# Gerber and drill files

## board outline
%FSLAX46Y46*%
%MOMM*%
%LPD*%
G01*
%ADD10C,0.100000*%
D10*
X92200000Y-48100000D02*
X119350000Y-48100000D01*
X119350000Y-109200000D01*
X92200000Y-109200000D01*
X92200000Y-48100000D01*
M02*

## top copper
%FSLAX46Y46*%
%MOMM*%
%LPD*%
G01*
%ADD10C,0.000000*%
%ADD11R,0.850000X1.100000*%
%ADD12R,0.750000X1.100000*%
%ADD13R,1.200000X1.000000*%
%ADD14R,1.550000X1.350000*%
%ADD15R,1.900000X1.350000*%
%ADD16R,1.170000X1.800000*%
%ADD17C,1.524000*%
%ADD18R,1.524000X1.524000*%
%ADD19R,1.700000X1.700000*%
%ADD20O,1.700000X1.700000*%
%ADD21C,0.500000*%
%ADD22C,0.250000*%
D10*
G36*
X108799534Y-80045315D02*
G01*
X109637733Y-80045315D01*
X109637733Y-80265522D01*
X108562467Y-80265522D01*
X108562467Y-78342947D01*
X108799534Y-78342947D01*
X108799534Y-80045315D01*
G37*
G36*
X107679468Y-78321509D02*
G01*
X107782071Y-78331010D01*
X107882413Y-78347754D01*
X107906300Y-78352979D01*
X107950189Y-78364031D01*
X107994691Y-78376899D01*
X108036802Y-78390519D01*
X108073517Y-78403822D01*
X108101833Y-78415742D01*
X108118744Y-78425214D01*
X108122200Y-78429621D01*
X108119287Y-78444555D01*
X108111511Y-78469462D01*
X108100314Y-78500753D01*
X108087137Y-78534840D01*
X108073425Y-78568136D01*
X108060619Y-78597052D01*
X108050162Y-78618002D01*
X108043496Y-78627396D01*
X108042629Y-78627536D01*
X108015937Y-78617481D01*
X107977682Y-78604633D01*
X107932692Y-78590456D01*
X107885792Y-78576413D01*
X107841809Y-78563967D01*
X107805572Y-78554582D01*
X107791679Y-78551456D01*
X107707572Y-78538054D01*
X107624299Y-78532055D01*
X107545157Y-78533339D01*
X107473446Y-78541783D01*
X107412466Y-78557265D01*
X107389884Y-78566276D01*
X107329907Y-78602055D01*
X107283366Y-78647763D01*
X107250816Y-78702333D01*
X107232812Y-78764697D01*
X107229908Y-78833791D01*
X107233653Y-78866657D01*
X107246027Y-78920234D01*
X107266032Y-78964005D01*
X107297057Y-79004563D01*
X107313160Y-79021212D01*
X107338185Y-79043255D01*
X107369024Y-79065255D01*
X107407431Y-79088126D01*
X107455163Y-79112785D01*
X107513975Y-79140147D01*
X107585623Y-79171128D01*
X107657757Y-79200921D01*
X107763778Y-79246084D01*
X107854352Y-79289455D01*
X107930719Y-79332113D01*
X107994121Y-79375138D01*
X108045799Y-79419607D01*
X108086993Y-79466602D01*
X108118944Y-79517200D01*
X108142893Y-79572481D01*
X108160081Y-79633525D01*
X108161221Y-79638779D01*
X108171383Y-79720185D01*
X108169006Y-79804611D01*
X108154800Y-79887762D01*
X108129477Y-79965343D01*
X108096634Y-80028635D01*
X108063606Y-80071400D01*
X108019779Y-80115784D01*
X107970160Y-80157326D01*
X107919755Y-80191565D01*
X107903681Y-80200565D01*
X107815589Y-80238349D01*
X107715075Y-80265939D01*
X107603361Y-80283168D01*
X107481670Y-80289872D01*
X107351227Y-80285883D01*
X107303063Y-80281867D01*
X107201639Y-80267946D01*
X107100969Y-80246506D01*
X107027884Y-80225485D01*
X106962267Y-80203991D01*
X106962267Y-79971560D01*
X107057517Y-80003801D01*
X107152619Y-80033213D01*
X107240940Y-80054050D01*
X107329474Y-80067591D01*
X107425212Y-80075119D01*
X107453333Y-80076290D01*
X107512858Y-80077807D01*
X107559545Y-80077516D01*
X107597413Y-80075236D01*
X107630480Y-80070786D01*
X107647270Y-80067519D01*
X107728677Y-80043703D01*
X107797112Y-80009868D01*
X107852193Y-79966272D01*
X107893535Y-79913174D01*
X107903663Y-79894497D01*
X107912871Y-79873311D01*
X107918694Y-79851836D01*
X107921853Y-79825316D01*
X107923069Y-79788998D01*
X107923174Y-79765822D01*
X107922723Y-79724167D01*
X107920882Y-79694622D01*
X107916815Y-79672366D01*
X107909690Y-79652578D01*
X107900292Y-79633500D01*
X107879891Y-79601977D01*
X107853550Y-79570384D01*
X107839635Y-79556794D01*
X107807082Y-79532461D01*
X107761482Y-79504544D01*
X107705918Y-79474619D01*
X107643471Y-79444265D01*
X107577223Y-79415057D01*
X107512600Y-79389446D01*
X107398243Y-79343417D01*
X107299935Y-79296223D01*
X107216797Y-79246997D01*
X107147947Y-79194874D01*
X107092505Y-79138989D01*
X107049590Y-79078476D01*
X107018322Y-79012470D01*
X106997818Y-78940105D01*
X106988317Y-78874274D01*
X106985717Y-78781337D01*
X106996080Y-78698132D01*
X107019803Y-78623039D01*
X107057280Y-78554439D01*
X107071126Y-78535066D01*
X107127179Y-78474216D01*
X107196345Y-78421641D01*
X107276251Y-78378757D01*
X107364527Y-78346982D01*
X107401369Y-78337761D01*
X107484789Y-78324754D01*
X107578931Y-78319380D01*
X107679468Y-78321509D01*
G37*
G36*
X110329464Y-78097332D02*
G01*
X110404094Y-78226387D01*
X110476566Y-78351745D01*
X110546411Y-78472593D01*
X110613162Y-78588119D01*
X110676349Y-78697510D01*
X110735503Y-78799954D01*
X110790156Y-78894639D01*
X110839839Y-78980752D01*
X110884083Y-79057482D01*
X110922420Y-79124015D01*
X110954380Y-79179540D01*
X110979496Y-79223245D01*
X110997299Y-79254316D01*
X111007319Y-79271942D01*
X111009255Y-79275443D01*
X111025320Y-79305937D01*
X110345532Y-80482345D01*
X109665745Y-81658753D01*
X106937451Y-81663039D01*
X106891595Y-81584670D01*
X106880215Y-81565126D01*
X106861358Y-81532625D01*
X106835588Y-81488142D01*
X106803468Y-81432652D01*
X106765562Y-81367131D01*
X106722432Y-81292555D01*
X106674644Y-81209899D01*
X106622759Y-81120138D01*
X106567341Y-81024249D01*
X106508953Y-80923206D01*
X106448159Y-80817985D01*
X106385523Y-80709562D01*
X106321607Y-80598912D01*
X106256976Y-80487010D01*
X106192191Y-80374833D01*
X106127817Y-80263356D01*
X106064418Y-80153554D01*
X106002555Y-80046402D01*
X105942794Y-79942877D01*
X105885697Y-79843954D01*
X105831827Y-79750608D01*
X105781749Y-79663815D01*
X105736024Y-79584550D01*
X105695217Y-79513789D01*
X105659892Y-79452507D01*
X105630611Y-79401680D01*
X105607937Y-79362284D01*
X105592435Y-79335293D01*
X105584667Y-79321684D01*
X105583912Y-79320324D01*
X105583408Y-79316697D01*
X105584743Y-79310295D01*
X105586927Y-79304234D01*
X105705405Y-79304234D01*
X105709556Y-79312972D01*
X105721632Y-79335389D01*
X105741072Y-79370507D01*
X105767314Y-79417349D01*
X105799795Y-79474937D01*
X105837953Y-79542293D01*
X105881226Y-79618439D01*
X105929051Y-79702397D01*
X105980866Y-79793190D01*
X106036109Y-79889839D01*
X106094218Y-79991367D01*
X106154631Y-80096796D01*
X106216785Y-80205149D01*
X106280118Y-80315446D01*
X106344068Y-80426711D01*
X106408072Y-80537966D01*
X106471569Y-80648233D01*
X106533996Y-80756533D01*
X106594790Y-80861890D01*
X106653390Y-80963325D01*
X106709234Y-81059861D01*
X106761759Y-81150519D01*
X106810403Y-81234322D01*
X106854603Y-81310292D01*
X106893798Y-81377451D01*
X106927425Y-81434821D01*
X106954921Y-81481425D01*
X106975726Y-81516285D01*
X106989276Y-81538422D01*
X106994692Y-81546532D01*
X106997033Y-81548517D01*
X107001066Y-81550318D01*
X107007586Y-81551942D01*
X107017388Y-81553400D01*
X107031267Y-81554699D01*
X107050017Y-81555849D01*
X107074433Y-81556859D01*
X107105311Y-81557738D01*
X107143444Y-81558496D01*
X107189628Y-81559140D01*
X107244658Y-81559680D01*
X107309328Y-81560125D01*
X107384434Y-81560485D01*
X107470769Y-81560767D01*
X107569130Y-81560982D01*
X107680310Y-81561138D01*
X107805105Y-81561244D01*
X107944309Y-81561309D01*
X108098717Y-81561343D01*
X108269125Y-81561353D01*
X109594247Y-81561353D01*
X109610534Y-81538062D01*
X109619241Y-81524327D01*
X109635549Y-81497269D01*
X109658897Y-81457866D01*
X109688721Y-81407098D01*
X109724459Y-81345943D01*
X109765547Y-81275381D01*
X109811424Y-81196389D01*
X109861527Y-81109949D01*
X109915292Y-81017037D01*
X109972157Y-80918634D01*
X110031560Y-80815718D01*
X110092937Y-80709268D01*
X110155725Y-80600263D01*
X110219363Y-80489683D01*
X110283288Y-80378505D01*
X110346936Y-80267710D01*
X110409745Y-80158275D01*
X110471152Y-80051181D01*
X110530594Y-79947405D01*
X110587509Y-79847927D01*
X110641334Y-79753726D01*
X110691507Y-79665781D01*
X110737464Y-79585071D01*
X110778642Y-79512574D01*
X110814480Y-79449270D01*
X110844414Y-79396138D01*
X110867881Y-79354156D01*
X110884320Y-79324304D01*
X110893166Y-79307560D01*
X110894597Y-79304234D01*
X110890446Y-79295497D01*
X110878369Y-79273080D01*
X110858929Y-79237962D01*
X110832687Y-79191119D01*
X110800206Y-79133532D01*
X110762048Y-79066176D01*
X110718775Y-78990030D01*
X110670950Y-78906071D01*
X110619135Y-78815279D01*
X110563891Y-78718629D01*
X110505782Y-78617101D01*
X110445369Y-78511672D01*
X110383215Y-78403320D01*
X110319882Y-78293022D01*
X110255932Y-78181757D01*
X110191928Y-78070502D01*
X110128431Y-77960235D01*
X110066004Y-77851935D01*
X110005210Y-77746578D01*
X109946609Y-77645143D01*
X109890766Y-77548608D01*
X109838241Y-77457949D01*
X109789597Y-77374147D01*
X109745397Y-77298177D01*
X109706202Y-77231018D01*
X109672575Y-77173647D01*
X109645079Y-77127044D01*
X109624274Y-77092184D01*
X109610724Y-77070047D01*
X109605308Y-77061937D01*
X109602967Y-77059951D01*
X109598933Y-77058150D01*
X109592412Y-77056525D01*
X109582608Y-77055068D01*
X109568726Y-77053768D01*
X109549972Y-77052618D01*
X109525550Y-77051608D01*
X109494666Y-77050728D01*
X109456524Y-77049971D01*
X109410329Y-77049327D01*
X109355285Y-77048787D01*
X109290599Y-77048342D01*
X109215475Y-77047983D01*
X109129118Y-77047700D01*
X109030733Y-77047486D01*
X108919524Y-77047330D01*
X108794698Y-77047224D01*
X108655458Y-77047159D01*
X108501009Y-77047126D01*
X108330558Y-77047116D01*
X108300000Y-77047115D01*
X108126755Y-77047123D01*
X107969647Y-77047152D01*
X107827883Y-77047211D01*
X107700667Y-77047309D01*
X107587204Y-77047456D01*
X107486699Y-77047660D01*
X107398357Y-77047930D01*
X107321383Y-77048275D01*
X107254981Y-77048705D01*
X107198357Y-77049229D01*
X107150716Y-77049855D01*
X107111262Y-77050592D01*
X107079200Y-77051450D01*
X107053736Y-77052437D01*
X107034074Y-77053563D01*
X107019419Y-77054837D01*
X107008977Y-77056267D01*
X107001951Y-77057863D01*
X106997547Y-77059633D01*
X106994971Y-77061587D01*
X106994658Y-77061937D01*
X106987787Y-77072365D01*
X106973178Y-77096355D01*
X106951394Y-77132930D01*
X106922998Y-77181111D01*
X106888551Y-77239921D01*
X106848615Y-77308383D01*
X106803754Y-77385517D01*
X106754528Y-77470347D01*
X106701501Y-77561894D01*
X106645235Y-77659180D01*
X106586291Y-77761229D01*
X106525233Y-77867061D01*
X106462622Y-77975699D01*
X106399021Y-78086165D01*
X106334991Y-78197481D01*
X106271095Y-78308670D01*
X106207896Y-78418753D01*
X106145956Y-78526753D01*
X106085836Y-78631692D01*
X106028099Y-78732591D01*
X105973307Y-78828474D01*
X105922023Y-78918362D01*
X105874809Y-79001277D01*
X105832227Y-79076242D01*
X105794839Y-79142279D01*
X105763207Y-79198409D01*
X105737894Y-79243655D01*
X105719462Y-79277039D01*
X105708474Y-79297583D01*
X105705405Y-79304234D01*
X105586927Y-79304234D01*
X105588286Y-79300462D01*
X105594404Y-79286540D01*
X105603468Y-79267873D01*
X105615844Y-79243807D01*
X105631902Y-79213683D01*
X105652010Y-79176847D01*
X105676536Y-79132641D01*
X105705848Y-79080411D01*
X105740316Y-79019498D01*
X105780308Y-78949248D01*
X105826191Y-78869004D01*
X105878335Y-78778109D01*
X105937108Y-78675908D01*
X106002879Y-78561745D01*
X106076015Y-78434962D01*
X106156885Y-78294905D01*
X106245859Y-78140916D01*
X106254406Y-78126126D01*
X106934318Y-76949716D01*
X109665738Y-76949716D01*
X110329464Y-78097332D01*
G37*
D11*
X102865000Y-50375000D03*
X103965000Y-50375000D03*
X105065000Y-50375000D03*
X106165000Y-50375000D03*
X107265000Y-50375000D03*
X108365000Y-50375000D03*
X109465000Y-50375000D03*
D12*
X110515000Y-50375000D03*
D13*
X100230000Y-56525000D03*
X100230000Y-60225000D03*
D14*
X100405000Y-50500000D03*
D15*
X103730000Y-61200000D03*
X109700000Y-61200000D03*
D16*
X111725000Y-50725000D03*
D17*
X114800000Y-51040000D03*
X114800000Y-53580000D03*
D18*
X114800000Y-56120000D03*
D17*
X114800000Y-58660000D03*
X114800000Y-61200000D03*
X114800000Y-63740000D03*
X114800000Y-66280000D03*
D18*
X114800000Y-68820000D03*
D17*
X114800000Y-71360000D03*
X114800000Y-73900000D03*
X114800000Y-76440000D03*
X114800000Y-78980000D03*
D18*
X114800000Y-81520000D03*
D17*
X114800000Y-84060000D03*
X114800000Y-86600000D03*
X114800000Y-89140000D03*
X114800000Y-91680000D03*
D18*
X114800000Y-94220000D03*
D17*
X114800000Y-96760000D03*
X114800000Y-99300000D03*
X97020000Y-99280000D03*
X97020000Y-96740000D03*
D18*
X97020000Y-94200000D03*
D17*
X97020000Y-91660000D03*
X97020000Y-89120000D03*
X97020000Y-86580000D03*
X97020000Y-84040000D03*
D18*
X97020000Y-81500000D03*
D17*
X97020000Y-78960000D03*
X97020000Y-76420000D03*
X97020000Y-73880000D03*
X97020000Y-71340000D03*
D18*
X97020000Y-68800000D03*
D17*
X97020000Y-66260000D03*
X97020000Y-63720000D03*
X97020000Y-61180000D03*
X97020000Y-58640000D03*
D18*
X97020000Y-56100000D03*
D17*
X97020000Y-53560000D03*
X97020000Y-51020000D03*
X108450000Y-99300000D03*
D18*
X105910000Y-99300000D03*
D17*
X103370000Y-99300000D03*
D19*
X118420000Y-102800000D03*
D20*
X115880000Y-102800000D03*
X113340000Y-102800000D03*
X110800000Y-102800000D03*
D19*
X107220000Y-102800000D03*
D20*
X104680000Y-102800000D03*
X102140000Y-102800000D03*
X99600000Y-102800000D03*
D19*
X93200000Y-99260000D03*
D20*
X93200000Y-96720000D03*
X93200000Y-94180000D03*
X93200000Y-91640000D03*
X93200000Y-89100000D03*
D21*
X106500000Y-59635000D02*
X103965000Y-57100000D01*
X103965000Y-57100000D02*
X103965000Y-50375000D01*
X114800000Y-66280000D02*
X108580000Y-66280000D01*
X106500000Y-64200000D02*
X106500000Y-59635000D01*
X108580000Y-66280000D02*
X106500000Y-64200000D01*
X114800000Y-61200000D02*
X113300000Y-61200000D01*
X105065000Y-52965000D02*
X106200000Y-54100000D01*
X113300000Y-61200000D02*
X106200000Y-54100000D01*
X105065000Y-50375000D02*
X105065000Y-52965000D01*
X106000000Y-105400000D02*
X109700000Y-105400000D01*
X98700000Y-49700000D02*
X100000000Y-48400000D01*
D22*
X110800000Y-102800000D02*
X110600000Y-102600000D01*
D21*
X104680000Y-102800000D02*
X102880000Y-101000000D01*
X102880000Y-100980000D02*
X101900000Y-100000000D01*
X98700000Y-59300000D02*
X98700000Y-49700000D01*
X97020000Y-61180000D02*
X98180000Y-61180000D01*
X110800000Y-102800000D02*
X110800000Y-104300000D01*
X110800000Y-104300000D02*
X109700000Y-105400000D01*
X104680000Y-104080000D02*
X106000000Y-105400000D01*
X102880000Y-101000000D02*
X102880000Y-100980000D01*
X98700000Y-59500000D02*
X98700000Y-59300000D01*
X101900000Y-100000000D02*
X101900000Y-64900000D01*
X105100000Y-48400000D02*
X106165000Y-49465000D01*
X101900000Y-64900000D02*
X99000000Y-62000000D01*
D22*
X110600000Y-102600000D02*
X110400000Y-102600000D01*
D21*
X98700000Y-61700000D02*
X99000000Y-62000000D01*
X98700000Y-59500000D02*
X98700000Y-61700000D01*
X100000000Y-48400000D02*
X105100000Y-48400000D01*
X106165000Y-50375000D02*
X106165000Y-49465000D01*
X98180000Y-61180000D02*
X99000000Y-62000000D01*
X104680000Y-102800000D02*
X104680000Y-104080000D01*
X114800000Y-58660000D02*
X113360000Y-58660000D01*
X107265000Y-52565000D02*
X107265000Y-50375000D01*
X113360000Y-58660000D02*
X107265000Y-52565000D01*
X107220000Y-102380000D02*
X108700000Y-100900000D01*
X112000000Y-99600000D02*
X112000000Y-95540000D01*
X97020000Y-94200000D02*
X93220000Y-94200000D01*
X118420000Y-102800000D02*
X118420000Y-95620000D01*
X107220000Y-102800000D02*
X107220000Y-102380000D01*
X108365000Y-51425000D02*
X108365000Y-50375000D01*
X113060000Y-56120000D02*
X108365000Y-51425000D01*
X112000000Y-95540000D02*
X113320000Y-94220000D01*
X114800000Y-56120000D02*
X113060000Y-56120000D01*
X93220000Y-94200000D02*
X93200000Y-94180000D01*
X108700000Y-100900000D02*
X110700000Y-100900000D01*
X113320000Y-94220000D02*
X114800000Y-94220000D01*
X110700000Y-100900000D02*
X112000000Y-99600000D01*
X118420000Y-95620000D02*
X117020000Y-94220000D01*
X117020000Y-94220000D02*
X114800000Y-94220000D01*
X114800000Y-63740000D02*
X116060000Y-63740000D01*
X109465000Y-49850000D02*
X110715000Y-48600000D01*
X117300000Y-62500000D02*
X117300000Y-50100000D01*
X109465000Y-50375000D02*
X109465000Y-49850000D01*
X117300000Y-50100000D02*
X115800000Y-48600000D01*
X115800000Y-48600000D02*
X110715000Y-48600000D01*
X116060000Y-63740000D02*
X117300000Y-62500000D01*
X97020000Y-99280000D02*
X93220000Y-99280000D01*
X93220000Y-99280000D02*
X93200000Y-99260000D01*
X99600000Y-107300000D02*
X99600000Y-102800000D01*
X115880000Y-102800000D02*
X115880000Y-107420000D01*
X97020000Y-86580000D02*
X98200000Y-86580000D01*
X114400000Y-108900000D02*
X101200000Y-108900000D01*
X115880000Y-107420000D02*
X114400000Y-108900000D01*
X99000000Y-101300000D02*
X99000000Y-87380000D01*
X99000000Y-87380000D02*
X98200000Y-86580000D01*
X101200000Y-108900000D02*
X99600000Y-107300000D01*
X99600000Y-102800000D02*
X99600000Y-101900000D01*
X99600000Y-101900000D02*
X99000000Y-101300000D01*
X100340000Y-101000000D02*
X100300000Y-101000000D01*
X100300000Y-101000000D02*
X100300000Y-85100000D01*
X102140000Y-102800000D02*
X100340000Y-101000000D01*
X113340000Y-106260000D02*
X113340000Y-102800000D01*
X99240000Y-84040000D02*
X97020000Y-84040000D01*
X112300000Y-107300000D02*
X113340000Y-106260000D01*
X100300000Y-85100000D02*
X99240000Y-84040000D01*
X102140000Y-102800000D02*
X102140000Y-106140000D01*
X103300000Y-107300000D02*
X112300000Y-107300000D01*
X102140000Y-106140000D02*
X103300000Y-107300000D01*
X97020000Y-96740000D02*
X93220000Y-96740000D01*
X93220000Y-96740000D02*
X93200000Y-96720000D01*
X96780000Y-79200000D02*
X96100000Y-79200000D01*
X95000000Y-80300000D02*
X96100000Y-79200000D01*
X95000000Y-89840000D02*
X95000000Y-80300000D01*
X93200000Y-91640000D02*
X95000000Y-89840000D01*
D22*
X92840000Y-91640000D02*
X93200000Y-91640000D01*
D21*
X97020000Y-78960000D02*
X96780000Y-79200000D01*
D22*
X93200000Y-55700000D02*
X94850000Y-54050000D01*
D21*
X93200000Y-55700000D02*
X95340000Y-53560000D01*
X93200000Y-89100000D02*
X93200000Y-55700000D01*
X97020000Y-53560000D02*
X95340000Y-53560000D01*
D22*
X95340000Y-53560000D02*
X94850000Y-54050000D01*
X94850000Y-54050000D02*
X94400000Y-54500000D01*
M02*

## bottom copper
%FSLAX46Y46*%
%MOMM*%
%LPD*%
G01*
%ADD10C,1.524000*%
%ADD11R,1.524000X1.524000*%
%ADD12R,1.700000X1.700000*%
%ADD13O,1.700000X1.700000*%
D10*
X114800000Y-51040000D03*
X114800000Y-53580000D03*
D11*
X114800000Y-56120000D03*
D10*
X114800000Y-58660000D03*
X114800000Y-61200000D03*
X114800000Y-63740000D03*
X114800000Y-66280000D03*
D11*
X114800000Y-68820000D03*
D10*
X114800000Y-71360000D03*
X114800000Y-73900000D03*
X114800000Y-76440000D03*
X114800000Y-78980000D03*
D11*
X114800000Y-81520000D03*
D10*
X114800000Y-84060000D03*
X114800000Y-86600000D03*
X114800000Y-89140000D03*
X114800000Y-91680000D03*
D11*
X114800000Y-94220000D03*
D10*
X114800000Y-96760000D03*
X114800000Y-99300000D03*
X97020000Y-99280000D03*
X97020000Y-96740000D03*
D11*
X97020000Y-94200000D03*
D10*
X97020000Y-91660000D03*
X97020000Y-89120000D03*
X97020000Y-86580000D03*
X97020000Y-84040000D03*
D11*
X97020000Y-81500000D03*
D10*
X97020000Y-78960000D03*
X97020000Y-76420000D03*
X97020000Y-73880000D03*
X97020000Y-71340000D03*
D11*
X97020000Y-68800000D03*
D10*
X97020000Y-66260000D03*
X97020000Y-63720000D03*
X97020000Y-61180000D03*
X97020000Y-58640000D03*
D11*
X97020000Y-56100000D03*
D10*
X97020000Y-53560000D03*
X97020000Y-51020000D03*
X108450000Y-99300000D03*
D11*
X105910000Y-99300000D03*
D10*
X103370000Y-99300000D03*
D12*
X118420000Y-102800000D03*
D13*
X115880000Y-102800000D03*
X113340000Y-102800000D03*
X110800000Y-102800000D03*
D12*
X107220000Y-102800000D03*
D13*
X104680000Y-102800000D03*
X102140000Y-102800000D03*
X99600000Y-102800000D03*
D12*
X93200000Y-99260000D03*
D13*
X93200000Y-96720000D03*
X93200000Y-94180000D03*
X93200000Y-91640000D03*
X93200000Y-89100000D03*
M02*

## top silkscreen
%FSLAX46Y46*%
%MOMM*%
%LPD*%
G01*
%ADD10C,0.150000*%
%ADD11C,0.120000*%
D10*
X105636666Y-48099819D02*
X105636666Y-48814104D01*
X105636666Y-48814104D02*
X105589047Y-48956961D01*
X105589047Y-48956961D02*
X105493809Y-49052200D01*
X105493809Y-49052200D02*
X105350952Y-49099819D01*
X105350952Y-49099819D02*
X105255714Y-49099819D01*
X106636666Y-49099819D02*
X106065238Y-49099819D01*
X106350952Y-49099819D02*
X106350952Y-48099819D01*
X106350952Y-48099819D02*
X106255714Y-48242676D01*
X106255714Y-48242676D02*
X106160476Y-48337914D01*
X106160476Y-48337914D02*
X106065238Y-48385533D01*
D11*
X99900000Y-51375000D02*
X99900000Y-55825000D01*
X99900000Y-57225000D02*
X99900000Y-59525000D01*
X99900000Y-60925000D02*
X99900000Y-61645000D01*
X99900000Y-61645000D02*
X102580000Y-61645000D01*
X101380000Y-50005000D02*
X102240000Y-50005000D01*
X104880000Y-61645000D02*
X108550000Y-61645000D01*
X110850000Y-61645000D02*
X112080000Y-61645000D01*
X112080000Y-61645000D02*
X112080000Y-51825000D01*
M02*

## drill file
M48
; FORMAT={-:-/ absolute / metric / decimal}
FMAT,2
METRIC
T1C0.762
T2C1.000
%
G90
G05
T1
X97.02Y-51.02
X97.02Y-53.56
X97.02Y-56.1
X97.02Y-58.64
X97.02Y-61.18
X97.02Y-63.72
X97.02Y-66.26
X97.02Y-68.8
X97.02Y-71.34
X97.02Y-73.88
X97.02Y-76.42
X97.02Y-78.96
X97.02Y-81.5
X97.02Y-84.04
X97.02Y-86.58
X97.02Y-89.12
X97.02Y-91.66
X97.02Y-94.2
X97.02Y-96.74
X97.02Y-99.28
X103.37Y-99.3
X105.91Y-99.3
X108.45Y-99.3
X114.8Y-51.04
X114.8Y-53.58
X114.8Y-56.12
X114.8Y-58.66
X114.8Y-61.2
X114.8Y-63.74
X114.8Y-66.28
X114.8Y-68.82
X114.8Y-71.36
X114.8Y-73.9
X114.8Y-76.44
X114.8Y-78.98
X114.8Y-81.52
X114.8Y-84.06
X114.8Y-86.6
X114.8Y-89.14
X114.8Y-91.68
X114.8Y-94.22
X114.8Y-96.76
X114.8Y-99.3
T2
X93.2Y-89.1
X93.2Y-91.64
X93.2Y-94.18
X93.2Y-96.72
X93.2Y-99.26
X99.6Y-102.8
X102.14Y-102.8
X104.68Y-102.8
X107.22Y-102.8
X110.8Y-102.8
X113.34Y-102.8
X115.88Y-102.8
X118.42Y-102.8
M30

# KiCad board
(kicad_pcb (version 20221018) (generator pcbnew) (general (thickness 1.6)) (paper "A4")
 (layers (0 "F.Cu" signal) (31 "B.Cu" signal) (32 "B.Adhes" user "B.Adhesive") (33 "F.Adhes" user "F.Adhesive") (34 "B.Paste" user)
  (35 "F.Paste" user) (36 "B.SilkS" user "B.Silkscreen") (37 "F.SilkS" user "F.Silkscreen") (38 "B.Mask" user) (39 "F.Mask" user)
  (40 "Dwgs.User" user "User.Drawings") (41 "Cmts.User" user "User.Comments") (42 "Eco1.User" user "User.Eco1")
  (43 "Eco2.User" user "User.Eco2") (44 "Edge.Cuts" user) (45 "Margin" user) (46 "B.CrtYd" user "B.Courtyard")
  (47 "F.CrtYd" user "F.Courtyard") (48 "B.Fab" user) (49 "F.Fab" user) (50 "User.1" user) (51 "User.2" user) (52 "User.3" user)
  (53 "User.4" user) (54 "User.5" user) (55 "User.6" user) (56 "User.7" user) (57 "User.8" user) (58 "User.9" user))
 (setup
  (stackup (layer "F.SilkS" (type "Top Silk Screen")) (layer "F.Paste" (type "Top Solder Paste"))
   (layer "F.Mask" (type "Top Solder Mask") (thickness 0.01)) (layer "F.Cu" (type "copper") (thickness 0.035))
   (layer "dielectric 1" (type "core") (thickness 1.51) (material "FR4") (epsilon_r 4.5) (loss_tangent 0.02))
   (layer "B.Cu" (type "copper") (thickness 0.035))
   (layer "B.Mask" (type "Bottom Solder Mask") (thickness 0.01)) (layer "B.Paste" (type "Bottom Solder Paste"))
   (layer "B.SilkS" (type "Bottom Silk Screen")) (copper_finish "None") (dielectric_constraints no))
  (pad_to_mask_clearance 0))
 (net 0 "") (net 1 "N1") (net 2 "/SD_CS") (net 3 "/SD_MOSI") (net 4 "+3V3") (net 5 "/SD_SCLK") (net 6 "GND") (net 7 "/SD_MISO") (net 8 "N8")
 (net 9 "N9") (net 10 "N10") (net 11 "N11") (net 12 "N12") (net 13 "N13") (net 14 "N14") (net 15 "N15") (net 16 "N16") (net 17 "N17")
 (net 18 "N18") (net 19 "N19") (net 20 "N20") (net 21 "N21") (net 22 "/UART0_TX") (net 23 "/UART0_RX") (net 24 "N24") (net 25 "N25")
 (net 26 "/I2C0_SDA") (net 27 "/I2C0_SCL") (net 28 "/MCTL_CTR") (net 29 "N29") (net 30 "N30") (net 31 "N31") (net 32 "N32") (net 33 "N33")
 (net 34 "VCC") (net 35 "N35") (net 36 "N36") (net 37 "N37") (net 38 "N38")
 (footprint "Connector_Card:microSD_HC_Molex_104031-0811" (layer "F.Cu") (at 105.97 55.825)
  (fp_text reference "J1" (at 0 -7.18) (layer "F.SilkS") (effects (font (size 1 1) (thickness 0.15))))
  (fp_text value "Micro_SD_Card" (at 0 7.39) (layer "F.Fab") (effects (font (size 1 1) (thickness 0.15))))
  (fp_line (start -6.07 -4.45) (end -6.07 0) (stroke (width 0.12) (type solid)) (layer "F.SilkS"))
  (fp_line (start -6.07 1.4) (end -6.07 3.7) (stroke (width 0.12) (type solid)) (layer "F.SilkS"))
  (fp_line (start -6.07 5.1) (end -6.07 5.82) (stroke (width 0.12) (type solid)) (layer "F.SilkS"))
  (fp_line (start -6.07 5.82) (end -3.39 5.82) (stroke (width 0.12) (type solid)) (layer "F.SilkS"))
  (fp_line (start -4.59 -5.82) (end -3.73 -5.82) (stroke (width 0.12) (type solid)) (layer "F.SilkS"))
  (fp_line (start -1.09 5.82) (end 2.58 5.82) (stroke (width 0.12) (type solid)) (layer "F.SilkS"))
  (fp_line (start 4.88 5.82) (end 6.11 5.82) (stroke (width 0.12) (type solid)) (layer "F.SilkS"))
  (fp_line (start 6.11 5.82) (end 6.11 -4) (stroke (width 0.12) (type solid)) (layer "F.SilkS"))
  (pad "1" smd rect (at -3.105 -5.45) (size 0.85 1.1) (layers "F.Cu" "F.Paste" "F.Mask") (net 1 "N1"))
  (pad "2" smd rect (at -2.005 -5.45) (size 0.85 1.1) (layers "F.Cu" "F.Paste" "F.Mask") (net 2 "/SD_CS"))
  (pad "3" smd rect (at -0.905 -5.45) (size 0.85 1.1) (layers "F.Cu" "F.Paste" "F.Mask") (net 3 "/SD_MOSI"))
  (pad "4" smd rect (at 0.195 -5.45) (size 0.85 1.1) (layers "F.Cu" "F.Paste" "F.Mask") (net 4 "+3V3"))
  (pad "5" smd rect (at 1.295 -5.45) (size 0.85 1.1) (layers "F.Cu" "F.Paste" "F.Mask") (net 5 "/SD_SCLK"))
  (pad "6" smd rect (at 2.395 -5.45) (size 0.85 1.1) (layers "F.Cu" "F.Paste" "F.Mask") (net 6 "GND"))
  (pad "7" smd rect (at 3.495 -5.45) (size 0.85 1.1) (layers "F.Cu" "F.Paste" "F.Mask") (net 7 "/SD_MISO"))
  (pad "8" smd rect (at 4.545 -5.45) (size 0.75 1.1) (layers "F.Cu" "F.Paste" "F.Mask") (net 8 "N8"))
  (pad "9" smd rect (at -5.74 0.7) (size 1.2 1) (layers "F.Cu" "F.Paste" "F.Mask") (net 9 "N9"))
  (pad "10" smd rect (at -5.74 4.4) (size 1.2 1) (layers "F.Cu" "F.Paste" "F.Mask"))
  (pad "11" smd rect (at -5.565 -5.325) (size 1.55 1.35) (layers "F.Cu" "F.Paste" "F.Mask"))
  (pad "11" smd rect (at -2.24 5.375) (size 1.9 1.35) (layers "F.Cu" "F.Paste" "F.Mask"))
  (pad "11" smd rect (at 3.73 5.375) (size 1.9 1.35) (layers "F.Cu" "F.Paste" "F.Mask"))
  (pad "11" smd rect (at 5.755 -5.1) (size 1.17 1.8) (layers "F.Cu" "F.Paste" "F.Mask")))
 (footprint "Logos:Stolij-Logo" (layer "F.Cu") (at 108.3 79.3) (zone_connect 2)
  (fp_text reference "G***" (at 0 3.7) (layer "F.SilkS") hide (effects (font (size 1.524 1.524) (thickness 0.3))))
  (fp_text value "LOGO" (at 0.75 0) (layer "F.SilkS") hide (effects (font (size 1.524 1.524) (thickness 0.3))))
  (fp_poly
   (pts (xy 0.499534 0.745315) (xy 1.337733 0.745315) (xy 1.337733 0.965522) (xy 0.262467 0.965522) (xy 0.262467 -0.957053)
    (xy 0.499534 -0.957053))
   (stroke (width 0) (type solid)) (fill solid) (layer "F.Cu"))
  (fp_poly
   (pts (xy -0.620532 -0.978491) (xy -0.517929 -0.96899) (xy -0.417587 -0.952246) (xy -0.3937 -0.947021) (xy -0.349811 -0.935969)
    (xy -0.305309 -0.923101) (xy -0.263198 -0.909481) (xy -0.226483 -0.896178) (xy -0.198167 -0.884258) (xy -0.181256 -0.874786)
    (xy -0.1778 -0.870379) (xy -0.180713 -0.855445) (xy -0.188489 -0.830538) (xy -0.199686 -0.799247) (xy -0.212863 -0.76516)
    (xy -0.226575 -0.731864) (xy -0.239381 -0.702948) (xy -0.249838 -0.681998) (xy -0.256504 -0.672604) (xy -0.257371 -0.672464)
    (xy -0.284063 -0.682519) (xy -0.322318 -0.695367) (xy -0.367308 -0.709544) (xy -0.414208 -0.723587) (xy -0.458191 -0.736033)
    (xy -0.494428 -0.745418) (xy -0.508321 -0.748544) (xy -0.592428 -0.761946) (xy -0.675701 -0.767945) (xy -0.754843 -0.766661)
    (xy -0.826554 -0.758217) (xy -0.887534 -0.742735) (xy -0.910116 -0.733724) (xy -0.970093 -0.697945) (xy -1.016634 -0.652237)
    (xy -1.049184 -0.597667) (xy -1.067188 -0.535303) (xy -1.070092 -0.466209) (xy -1.066347 -0.433343) (xy -1.053973 -0.379766)
    (xy -1.033968 -0.335995) (xy -1.002943 -0.295437) (xy -0.98684 -0.278788) (xy -0.961815 -0.256745) (xy -0.930976 -0.234745)
    (xy -0.892569 -0.211874) (xy -0.844837 -0.187215) (xy -0.786025 -0.159853) (xy -0.714377 -0.128872) (xy -0.642243 -0.099079)
    (xy -0.536222 -0.053916) (xy -0.445648 -0.010545) (xy -0.369281 0.032113) (xy -0.305879 0.075138) (xy -0.254201 0.119607)
    (xy -0.213007 0.166602) (xy -0.181056 0.2172) (xy -0.157107 0.272481) (xy -0.139919 0.333525) (xy -0.138779 0.338779)
    (xy -0.128617 0.420185) (xy -0.130994 0.504611) (xy -0.1452 0.587762) (xy -0.170523 0.665343) (xy -0.203366 0.728635)
    (xy -0.236394 0.7714) (xy -0.280221 0.815784) (xy -0.32984 0.857326) (xy -0.380245 0.891565) (xy -0.396319 0.900565)
    (xy -0.484411 0.938349) (xy -0.584925 0.965939) (xy -0.696639 0.983168) (xy -0.81833 0.989872) (xy -0.948773 0.985883)
    (xy -0.996937 0.981867) (xy -1.098361 0.967946) (xy -1.199031 0.946506) (xy -1.272116 0.925485) (xy -1.337733 0.903991)
    (xy -1.337733 0.67156) (xy -1.242483 0.703801) (xy -1.147381 0.733213) (xy -1.05906 0.75405) (xy -0.970526 0.767591)
    (xy -0.874788 0.775119) (xy -0.846667 0.77629) (xy -0.787142 0.777807) (xy -0.740455 0.777516) (xy -0.702587 0.775236)
    (xy -0.66952 0.770786) (xy -0.65273 0.767519) (xy -0.571323 0.743703) (xy -0.502888 0.709868) (xy -0.447807 0.666272)
    (xy -0.406465 0.613174) (xy -0.396337 0.594497) (xy -0.387129 0.573311) (xy -0.381306 0.551836) (xy -0.378147 0.525316)
    (xy -0.376931 0.488998) (xy -0.376826 0.465822) (xy -0.377277 0.424167) (xy -0.379118 0.394622) (xy -0.383185 0.372366)
    (xy -0.39031 0.352578) (xy -0.399708 0.3335) (xy -0.420109 0.301977) (xy -0.44645 0.270384) (xy -0.460365 0.256794)
    (xy -0.492918 0.232461) (xy -0.538518 0.204544) (xy -0.594082 0.174619) (xy -0.656529 0.144265) (xy -0.722777 0.115057)
    (xy -0.7874 0.089446) (xy -0.901757 0.043417) (xy -1.000065 -0.003777) (xy -1.083203 -0.053003) (xy -1.152053 -0.105126)
    (xy -1.207495 -0.161011) (xy -1.25041 -0.221524) (xy -1.281678 -0.28753) (xy -1.302182 -0.359895) (xy -1.311683 -0.425726)
    (xy -1.314283 -0.518663) (xy -1.30392 -0.601868) (xy -1.280197 -0.676961) (xy -1.24272 -0.745561) (xy -1.228874 -0.764934)
    (xy -1.172821 -0.825784) (xy -1.103655 -0.878359) (xy -1.023749 -0.921243) (xy -0.935473 -0.953018) (xy -0.898631 -0.962239)
    (xy -0.815211 -0.975246) (xy -0.721069 -0.98062))
   (stroke (width 0) (type solid)) (fill solid) (layer "F.Cu"))
  (fp_poly
   (pts (xy 2.029464 -1.202668) (xy 2.104094 -1.073613) (xy 2.176566 -0.948255) (xy 2.246411 -0.827407) (xy 2.313162 -0.711881)
    (xy 2.376349 -0.60249) (xy 2.435503 -0.500046) (xy 2.490156 -0.405361) (xy 2.539839 -0.319248) (xy 2.584083 -0.242518)
    (xy 2.62242 -0.175985) (xy 2.65438 -0.12046) (xy 2.679496 -0.076755) (xy 2.697299 -0.045684) (xy 2.707319 -0.028058)
    (xy 2.709255 -0.024557) (xy 2.72532 0.005937) (xy 2.045532 1.182345) (xy 1.365745 2.358753) (xy -1.362549 2.363039)
    (xy -1.408405 2.28467) (xy -1.419785 2.265126) (xy -1.438642 2.232625) (xy -1.464412 2.188142) (xy -1.496532 2.132652)
    (xy -1.534438 2.067131) (xy -1.577568 1.992555) (xy -1.625356 1.909899) (xy -1.677241 1.820138) (xy -1.732659 1.724249)
    (xy -1.791047 1.623206) (xy -1.851841 1.517985) (xy -1.914477 1.409562) (xy -1.978393 1.298912) (xy -2.043024 1.18701)
    (xy -2.107809 1.074833) (xy -2.172183 0.963356) (xy -2.235582 0.853554) (xy -2.297445 0.746402) (xy -2.357206 0.642877)
    (xy -2.414303 0.543954) (xy -2.468173 0.450608) (xy -2.518251 0.363815) (xy -2.563976 0.28455) (xy -2.604783 0.213789)
    (xy -2.640108 0.152507) (xy -2.669389 0.10168) (xy -2.692063 0.062284) (xy -2.707565 0.035293) (xy -2.715333 0.021684)
    (xy -2.716088 0.020324) (xy -2.716592 0.016697) (xy -2.715257 0.010295) (xy -2.713073 0.004234) (xy -2.594595 0.004234)
    (xy -2.590444 0.012972) (xy -2.578368 0.035389) (xy -2.558928 0.070507) (xy -2.532686 0.117349) (xy -2.500205 0.174937)
    (xy -2.462047 0.242293) (xy -2.418774 0.318439) (xy -2.370949 0.402397) (xy -2.319134 0.49319) (xy -2.263891 0.589839)
    (xy -2.205782 0.691367) (xy -2.145369 0.796796) (xy -2.083215 0.905149) (xy -2.019882 1.015446) (xy -1.955932 1.126711)
    (xy -1.891928 1.237966) (xy -1.828431 1.348233) (xy -1.766004 1.456533) (xy -1.70521 1.56189) (xy -1.64661 1.663325)
    (xy -1.590766 1.759861) (xy -1.538241 1.850519) (xy -1.489597 1.934322) (xy -1.445397 2.010292) (xy -1.406202 2.077451)
    (xy -1.372575 2.134821) (xy -1.345079 2.181425) (xy -1.324274 2.216285) (xy -1.310724 2.238422) (xy -1.305308 2.246532)
    (xy -1.302967 2.248517) (xy -1.298934 2.250318) (xy -1.292414 2.251942) (xy -1.282612 2.2534) (xy -1.268733 2.254699)
    (xy -1.249983 2.255849) (xy -1.225567 2.256859) (xy -1.194689 2.257738) (xy -1.156556 2.258496) (xy -1.110372 2.25914)
    (xy -1.055342 2.25968) (xy -0.990672 2.260125) (xy -0.915566 2.260485) (xy -0.829231 2.260767) (xy -0.73087 2.260982)
    (xy -0.61969 2.261138) (xy -0.494895 2.261244) (xy -0.355691 2.261309) (xy -0.201283 2.261343) (xy -0.030875 2.261353)
    (xy 1.294247 2.261353) (xy 1.310534 2.238062) (xy 1.319241 2.224327) (xy 1.335549 2.197269) (xy 1.358897 2.157866)
    (xy 1.388721 2.107098) (xy 1.424459 2.045943) (xy 1.465547 1.975381) (xy 1.511424 1.896389) (xy 1.561527 1.809949)
    (xy 1.615292 1.717037) (xy 1.672157 1.618634) (xy 1.73156 1.515718) (xy 1.792937 1.409268) (xy 1.855725 1.300263) (xy 1.919363 1.189683)
    (xy 1.983288 1.078505) (xy 2.046936 0.96771) (xy 2.109745 0.858275) (xy 2.171152 0.751181) (xy 2.230594 0.647405) (xy 2.287509 0.547927)
    (xy 2.341334 0.453726) (xy 2.391507 0.365781) (xy 2.437464 0.285071) (xy 2.478642 0.212574) (xy 2.51448 0.14927) (xy 2.544414 0.096138)
    (xy 2.567881 0.054156) (xy 2.58432 0.024304) (xy 2.593166 0.00756) (xy 2.594597 0.004234) (xy 2.590446 -0.004503) (xy 2.578369 -0.02692)
    (xy 2.558929 -0.062038) (xy 2.532687 -0.108881) (xy 2.500206 -0.166468) (xy 2.462048 -0.233824) (xy 2.418775 -0.30997)
    (xy 2.37095 -0.393929) (xy 2.319135 -0.484721) (xy 2.263891 -0.581371) (xy 2.205782 -0.682899) (xy 2.145369 -0.788328)
    (xy 2.083215 -0.89668) (xy 2.019882 -1.006978) (xy 1.955932 -1.118243) (xy 1.891928 -1.229498) (xy 1.828431 -1.339765)
    (xy 1.766004 -1.448065) (xy 1.70521 -1.553422) (xy 1.646609 -1.654857) (xy 1.590766 -1.751392) (xy 1.538241 -1.842051)
    (xy 1.489597 -1.925853) (xy 1.445397 -2.001823) (xy 1.406202 -2.068982) (xy 1.372575 -2.126353) (xy 1.345079 -2.172956)
    (xy 1.324274 -2.207816) (xy 1.310724 -2.229953) (xy 1.305308 -2.238063) (xy 1.302967 -2.240049) (xy 1.298933 -2.24185)
    (xy 1.292412 -2.243475) (xy 1.282608 -2.244932) (xy 1.268726 -2.246232) (xy 1.249972 -2.247382) (xy 1.22555 -2.248392)
    (xy 1.194666 -2.249272) (xy 1.156524 -2.250029) (xy 1.110329 -2.250673) (xy 1.055285 -2.251213) (xy 0.990599 -2.251658)
    (xy 0.915475 -2.252017) (xy 0.829118 -2.2523) (xy 0.730733 -2.252514) (xy 0.619524 -2.25267) (xy 0.494698 -2.252776)
    (xy 0.355458 -2.252841) (xy 0.201009 -2.252874) (xy 0.030558 -2.252884) (xy 0 -2.252885) (xy -0.173245 -2.252877)
    (xy -0.330353 -2.252848) (xy -0.472117 -2.252789) (xy -0.599333 -2.252691) (xy -0.712796 -2.252544) (xy -0.813301 -2.25234)
    (xy -0.901643 -2.25207) (xy -0.978617 -2.251725) (xy -1.045019 -2.251295) (xy -1.101643 -2.250771) (xy -1.149284 -2.250145)
    (xy -1.188738 -2.249408) (xy -1.2208 -2.24855) (xy -1.246264 -2.247563) (xy -1.265926 -2.246437) (xy -1.280581 -2.245163)
    (xy -1.291023 -2.243733) (xy -1.298049 -2.242137) (xy -1.302453 -2.240367) (xy -1.305029 -2.238413) (xy -1.305342 -2.238063)
    (xy -1.312213 -2.227635) (xy -1.326822 -2.203645) (xy -1.348606 -2.16707) (xy -1.377002 -2.118889) (xy -1.411449 -2.060079)
    (xy -1.451385 -1.991617) (xy -1.496246 -1.914483) (xy -1.545472 -1.829653) (xy -1.598499 -1.738106) (xy -1.654765 -1.64082)
    (xy -1.713709 -1.538771) (xy -1.774767 -1.432939) (xy -1.837378 -1.324301) (xy -1.900979 -1.213835) (xy -1.965009 -1.102519)
    (xy -2.028905 -0.99133) (xy -2.092104 -0.881247) (xy -2.154044 -0.773247) (xy -2.214164 -0.668308) (xy -2.271901 -0.567409)
    (xy -2.326693 -0.471526) (xy -2.377977 -0.381638) (xy -2.425191 -0.298723) (xy -2.467773 -0.223758) (xy -2.505161 -0.157721)
    (xy -2.536793 -0.101591) (xy -2.562106 -0.056345) (xy -2.580538 -0.022961) (xy -2.591526 -0.002417) (xy -2.594595 0.004234)
    (xy -2.713073 0.004234) (xy -2.711714 0.000462) (xy -2.705596 -0.01346) (xy -2.696532 -0.032127) (xy -2.684156 -0.056193)
    (xy -2.668098 -0.086317) (xy -2.64799 -0.123153) (xy -2.623464 -0.167359) (xy -2.594152 -0.219589) (xy -2.559684 -0.280502)
    (xy -2.519692 -0.350752) (xy -2.473809 -0.430996) (xy -2.421665 -0.521891) (xy -2.362892 -0.624092) (xy -2.297121 -0.738255)
    (xy -2.223985 -0.865038) (xy -2.143115 -1.005095) (xy -2.054141 -1.159084) (xy -2.045594 -1.173874) (xy -1.365682 -2.350284)
    (xy 1.365738 -2.350284))
   (stroke (width 0) (type solid)) (fill solid) (layer "F.Cu")))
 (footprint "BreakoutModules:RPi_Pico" (layer "B.Cu") (at 116.41 100.65 180)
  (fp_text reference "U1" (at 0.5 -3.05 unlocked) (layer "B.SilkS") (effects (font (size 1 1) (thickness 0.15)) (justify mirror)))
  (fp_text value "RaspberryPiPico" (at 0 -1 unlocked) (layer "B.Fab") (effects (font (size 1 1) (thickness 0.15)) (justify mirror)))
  (pad "1" thru_hole circle (at 1.61 49.61 180) (size 1.524 1.524) (drill 0.762) (layers "*.Cu" "*.Mask") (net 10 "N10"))
  (pad "2" thru_hole circle (at 1.61 47.07 180) (size 1.524 1.524) (drill 0.762) (layers "*.Cu" "*.Mask") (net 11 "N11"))
  (pad "3" thru_hole rect (at 1.61 44.53 180) (size 1.524 1.524) (drill 0.762) (layers "*.Cu" "*.Mask") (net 6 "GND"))
  (pad "4" thru_hole circle (at 1.61 41.99 180) (size 1.524 1.524) (drill 0.762) (layers "*.Cu" "*.Mask") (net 5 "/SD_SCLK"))
  (pad "5" thru_hole circle (at 1.61 39.45 180) (size 1.524 1.524) (drill 0.762) (layers "*.Cu" "*.Mask") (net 3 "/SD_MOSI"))
  (pad "6" thru_hole circle (at 1.61 36.91 180) (size 1.524 1.524) (drill 0.762) (layers "*.Cu" "*.Mask") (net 7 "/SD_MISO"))
  (pad "7" thru_hole circle (at 1.61 34.37 180) (size 1.524 1.524) (drill 0.762) (layers "*.Cu" "*.Mask") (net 2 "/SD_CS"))
  (pad "8" thru_hole rect (at 1.61 31.83 180) (size 1.524 1.524) (drill 0.762) (layers "*.Cu" "*.Mask") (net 6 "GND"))
  (pad "9" thru_hole circle (at 1.61 29.29 180) (size 1.524 1.524) (drill 0.762) (layers "*.Cu" "*.Mask") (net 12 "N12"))
  (pad "10" thru_hole circle (at 1.61 26.75 180) (size 1.524 1.524) (drill 0.762) (layers "*.Cu" "*.Mask") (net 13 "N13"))
  (pad "11" thru_hole circle (at 1.61 24.21 180) (size 1.524 1.524) (drill 0.762) (layers "*.Cu" "*.Mask") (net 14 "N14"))
  (pad "12" thru_hole circle (at 1.61 21.67 180) (size 1.524 1.524) (drill 0.762) (layers "*.Cu" "*.Mask") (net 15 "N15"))
  (pad "13" thru_hole rect (at 1.61 19.13 180) (size 1.524 1.524) (drill 0.762) (layers "*.Cu" "*.Mask") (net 6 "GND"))
  (pad "14" thru_hole circle (at 1.61 16.59 180) (size 1.524 1.524) (drill 0.762) (layers "*.Cu" "*.Mask") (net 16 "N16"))
  (pad "15" thru_hole circle (at 1.61 14.05 180) (size 1.524 1.524) (drill 0.762) (layers "*.Cu" "*.Mask") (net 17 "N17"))
  (pad "16" thru_hole circle (at 1.61 11.51 180) (size 1.524 1.524) (drill 0.762) (layers "*.Cu" "*.Mask") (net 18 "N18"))
  (pad "17" thru_hole circle (at 1.61 8.97 180) (size 1.524 1.524) (drill 0.762) (layers "*.Cu" "*.Mask") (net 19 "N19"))
  (pad "18" thru_hole rect (at 1.61 6.43 180) (size 1.524 1.524) (drill 0.762) (layers "*.Cu" "*.Mask") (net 6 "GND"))
  (pad "19" thru_hole circle (at 1.61 3.89 180) (size 1.524 1.524) (drill 0.762) (layers "*.Cu" "*.Mask") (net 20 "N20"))
  (pad "20" thru_hole circle (at 1.61 1.35 180) (size 1.524 1.524) (drill 0.762) (layers "*.Cu" "*.Mask") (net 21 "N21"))
  (pad "21" thru_hole circle (at 19.39 1.37 180) (size 1.524 1.524) (drill 0.762) (layers "*.Cu" "*.Mask") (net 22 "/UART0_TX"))
  (pad "22" thru_hole circle (at 19.39 3.91 180) (size 1.524 1.524) (drill 0.762) (layers "*.Cu" "*.Mask") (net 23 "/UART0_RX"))
  (pad "23" thru_hole rect (at 19.39 6.45 180) (size 1.524 1.524) (drill 0.762) (layers "*.Cu" "*.Mask") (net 6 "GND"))
  (pad "24" thru_hole circle (at 19.39 8.99 180) (size 1.524 1.524) (drill 0.762) (layers "*.Cu" "*.Mask") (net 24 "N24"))
  (pad "25" thru_hole circle (at 19.39 11.53 180) (size 1.524 1.524) (drill 0.762) (layers "*.Cu" "*.Mask") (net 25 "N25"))
  (pad "26" thru_hole circle (at 19.39 14.07 180) (size 1.524 1.524) (drill 0.762) (layers "*.Cu" "*.Mask") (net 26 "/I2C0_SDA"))
  (pad "27" thru_hole circle (at 19.39 16.61 180) (size 1.524 1.524) (drill 0.762) (layers "*.Cu" "*.Mask") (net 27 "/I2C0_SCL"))
  (pad "28" thru_hole rect (at 19.39 19.15 180) (size 1.524 1.524) (drill 0.762) (layers "*.Cu" "*.Mask") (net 6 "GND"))
  (pad "29" thru_hole circle (at 19.39 21.69 180) (size 1.524 1.524) (drill 0.762) (layers "*.Cu" "*.Mask") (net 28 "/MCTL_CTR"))
  (pad "30" thru_hole circle (at 19.39 24.23 180) (size 1.524 1.524) (drill 0.762) (layers "*.Cu" "*.Mask") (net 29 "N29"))
  (pad "31" thru_hole circle (at 19.39 26.77 180) (size 1.524 1.524) (drill 0.762) (layers "*.Cu" "*.Mask") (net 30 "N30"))
  (pad "32" thru_hole circle (at 19.39 29.31 180) (size 1.524 1.524) (drill 0.762) (layers "*.Cu" "*.Mask") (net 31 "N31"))
  (pad "33" thru_hole rect (at 19.39 31.85 180) (size 1.524 1.524) (drill 0.762) (layers "*.Cu" "*.Mask") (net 6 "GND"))
  (pad "34" thru_hole circle (at 19.39 34.39 180) (size 1.524 1.524) (drill 0.762) (layers "*.Cu" "*.Mask") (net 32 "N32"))
  (pad "35" thru_hole circle (at 19.39 36.93 180) (size 1.524 1.524) (drill 0.762) (layers "*.Cu" "*.Mask"))
  (pad "36" thru_hole circle (at 19.39 39.47 180) (size 1.524 1.524) (drill 0.762) (layers "*.Cu" "*.Mask") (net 4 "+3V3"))
  (pad "37" thru_hole circle (at 19.39 42.01 180) (size 1.524 1.524) (drill 0.762) (layers "*.Cu" "*.Mask") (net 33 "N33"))
  (pad "38" thru_hole rect (at 19.39 44.55 180) (size 1.524 1.524) (drill 0.762) (layers "*.Cu" "*.Mask") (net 6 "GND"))
  (pad "39" thru_hole circle (at 19.39 47.09 180) (size 1.524 1.524) (drill 0.762) (layers "*.Cu" "*.Mask") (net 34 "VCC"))
  (pad "40" thru_hole circle (at 19.39 49.63 180) (size 1.524 1.524) (drill 0.762) (layers "*.Cu" "*.Mask") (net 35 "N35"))
  (pad "41" thru_hole circle (at 7.96 1.35 180) (size 1.524 1.524) (drill 0.762) (layers "*.Cu" "*.Mask") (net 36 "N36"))
  (pad "42" thru_hole rect (at 10.5 1.35 180) (size 1.524 1.524) (drill 0.762) (layers "*.Cu" "*.Mask") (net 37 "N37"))
  (pad "43" thru_hole circle (at 13.04 1.35 180) (size 1.524 1.524) (drill 0.762) (layers "*.Cu" "*.Mask") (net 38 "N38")))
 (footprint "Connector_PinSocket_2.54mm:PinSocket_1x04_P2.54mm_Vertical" (layer "B.Cu") (at 118.42 102.8 90)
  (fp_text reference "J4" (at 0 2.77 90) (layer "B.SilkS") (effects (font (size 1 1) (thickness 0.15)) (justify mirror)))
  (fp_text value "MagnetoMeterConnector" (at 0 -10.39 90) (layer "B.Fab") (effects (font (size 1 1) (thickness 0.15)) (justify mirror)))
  (pad "1" thru_hole rect (at 0 0 90) (size 1.7 1.7) (drill 1) (layers "*.Cu" "*.Mask") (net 6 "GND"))
  (pad "2" thru_hole oval (at 0 -2.54 90) (size 1.7 1.7) (drill 1) (layers "*.Cu" "*.Mask") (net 26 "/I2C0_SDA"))
  (pad "3" thru_hole oval (at 0 -5.08 90) (size 1.7 1.7) (drill 1) (layers "*.Cu" "*.Mask") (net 27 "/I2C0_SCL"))
  (pad "4" thru_hole oval (at 0 -7.62 90) (size 1.7 1.7) (drill 1) (layers "*.Cu" "*.Mask") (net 4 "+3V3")))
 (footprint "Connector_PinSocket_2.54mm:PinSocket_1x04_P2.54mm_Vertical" (layer "B.Cu") (at 107.22 102.8 90)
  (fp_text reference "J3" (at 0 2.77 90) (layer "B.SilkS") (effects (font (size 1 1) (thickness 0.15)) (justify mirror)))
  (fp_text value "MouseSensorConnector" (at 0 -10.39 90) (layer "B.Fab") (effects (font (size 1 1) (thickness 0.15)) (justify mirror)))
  (pad "1" thru_hole rect (at 0 0 90) (size 1.7 1.7) (drill 1) (layers "*.Cu" "*.Mask") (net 6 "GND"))
  (pad "2" thru_hole oval (at 0 -2.54 90) (size 1.7 1.7) (drill 1) (layers "*.Cu" "*.Mask") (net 4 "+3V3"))
  (pad "3" thru_hole oval (at 0 -5.08 90) (size 1.7 1.7) (drill 1) (layers "*.Cu" "*.Mask") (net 27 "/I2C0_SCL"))
  (pad "4" thru_hole oval (at 0 -7.62 90) (size 1.7 1.7) (drill 1) (layers "*.Cu" "*.Mask") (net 26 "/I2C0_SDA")))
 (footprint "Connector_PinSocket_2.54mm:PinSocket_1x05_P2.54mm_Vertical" (layer "B.Cu") (at 93.2 99.26)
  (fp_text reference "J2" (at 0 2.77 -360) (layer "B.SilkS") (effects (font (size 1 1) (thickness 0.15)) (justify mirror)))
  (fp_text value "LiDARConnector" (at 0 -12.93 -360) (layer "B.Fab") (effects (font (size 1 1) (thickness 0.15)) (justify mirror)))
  (pad "1" thru_hole rect (at 0 0) (size 1.7 1.7) (drill 1) (layers "*.Cu" "*.Mask") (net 22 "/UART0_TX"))
  (pad "2" thru_hole oval (at 0 -2.54) (size 1.7 1.7) (drill 1) (layers "*.Cu" "*.Mask") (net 23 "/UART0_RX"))
  (pad "3" thru_hole oval (at 0 -5.08) (size 1.7 1.7) (drill 1) (layers "*.Cu" "*.Mask") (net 6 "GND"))
  (pad "4" thru_hole oval (at 0 -7.62) (size 1.7 1.7) (drill 1) (layers "*.Cu" "*.Mask") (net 28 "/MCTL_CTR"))
  (pad "5" thru_hole oval (at 0 -10.16) (size 1.7 1.7) (drill 1) (layers "*.Cu" "*.Mask") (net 34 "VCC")))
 (gr_rect (start 92.2 48.1) (end 119.35 109.2) (stroke (width 0.1) (type default)) (fill none) (layer "Edge.Cuts"))
 (segment (start 106.5 59.635) (end 103.965 57.1) (width 0.5) (layer "F.Cu") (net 2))
 (segment (start 103.965 57.1) (end 103.965 50.375) (width 0.5) (layer "F.Cu") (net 2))
 (segment (start 114.8 66.28) (end 108.58 66.28) (width 0.5) (layer "F.Cu") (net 2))
 (segment (start 106.5 64.2) (end 106.5 59.635) (width 0.5) (layer "F.Cu") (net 2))
 (segment (start 108.58 66.28) (end 106.5 64.2) (width 0.5) (layer "F.Cu") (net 2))
 (segment (start 114.8 61.2) (end 113.3 61.2) (width 0.5) (layer "F.Cu") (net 3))
 (segment (start 105.065 52.965) (end 106.2 54.1) (width 0.5) (layer "F.Cu") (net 3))
 (segment (start 113.3 61.2) (end 106.2 54.1) (width 0.5) (layer "F.Cu") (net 3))
 (segment (start 105.065 50.375) (end 105.065 52.965) (width 0.5) (layer "F.Cu") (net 3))
 (segment (start 106 105.4) (end 109.7 105.4) (width 0.5) (layer "F.Cu") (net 4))
 (segment (start 98.7 49.7) (end 100 48.4) (width 0.5) (layer "F.Cu") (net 4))
 (segment (start 110.8 102.8) (end 110.6 102.6) (width 0.25) (layer "F.Cu") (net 4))
 (segment (start 104.68 102.8) (end 102.88 101) (width 0.5) (layer "F.Cu") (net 4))
 (segment (start 102.88 100.98) (end 101.9 100) (width 0.5) (layer "F.Cu") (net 4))
 (segment (start 98.7 59.3) (end 98.7 49.7) (width 0.5) (layer "F.Cu") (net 4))
 (segment (start 97.02 61.18) (end 98.18 61.18) (width 0.5) (layer "F.Cu") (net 4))
 (segment (start 110.8 102.8) (end 110.8 104.3) (width 0.5) (layer "F.Cu") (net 4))
 (segment (start 110.8 104.3) (end 109.7 105.4) (width 0.5) (layer "F.Cu") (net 4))
 (segment (start 104.68 104.08) (end 106 105.4) (width 0.5) (layer "F.Cu") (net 4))
 (segment (start 102.88 101) (end 102.88 100.98) (width 0.5) (layer "F.Cu") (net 4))
 (segment (start 98.7 59.5) (end 98.7 59.3) (width 0.5) (layer "F.Cu") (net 4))
 (segment (start 101.9 100) (end 101.9 64.9) (width 0.5) (layer "F.Cu") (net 4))
 (segment (start 105.1 48.4) (end 106.165 49.465) (width 0.5) (layer "F.Cu") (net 4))
 (segment (start 101.9 64.9) (end 99 62) (width 0.5) (layer "F.Cu") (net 4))
 (segment (start 110.6 102.6) (end 110.4 102.6) (width 0.25) (layer "F.Cu") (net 4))
 (segment (start 98.7 61.7) (end 99 62) (width 0.5) (layer "F.Cu") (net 4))
 (segment (start 98.7 59.5) (end 98.7 61.7) (width 0.5) (layer "F.Cu") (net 4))
 (segment (start 100 48.4) (end 105.1 48.4) (width 0.5) (layer "F.Cu") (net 4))
 (segment (start 106.165 50.375) (end 106.165 49.465) (width 0.5) (layer "F.Cu") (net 4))
 (segment (start 98.18 61.18) (end 99 62) (width 0.5) (layer "F.Cu") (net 4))
 (segment (start 104.68 102.8) (end 104.68 104.08) (width 0.5) (layer "F.Cu") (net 4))
 (segment (start 114.8 58.66) (end 113.36 58.66) (width 0.5) (layer "F.Cu") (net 5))
 (segment (start 107.265 52.565) (end 107.265 50.375) (width 0.5) (layer "F.Cu") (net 5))
 (segment (start 113.36 58.66) (end 107.265 52.565) (width 0.5) (layer "F.Cu") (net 5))
 (segment (start 107.22 102.38) (end 108.7 100.9) (width 0.5) (layer "F.Cu") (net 6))
 (segment (start 112 99.6) (end 112 95.54) (width 0.5) (layer "F.Cu") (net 6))
 (segment (start 97.02 94.2) (end 93.22 94.2) (width 0.5) (layer "F.Cu") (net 6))
 (segment (start 118.42 102.8) (end 118.42 95.62) (width 0.5) (layer "F.Cu") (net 6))
 (segment (start 107.22 102.8) (end 107.22 102.38) (width 0.5) (layer "F.Cu") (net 6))
 (segment (start 108.365 51.425) (end 108.365 50.375) (width 0.5) (layer "F.Cu") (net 6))
 (segment (start 113.06 56.12) (end 108.365 51.425) (width 0.5) (layer "F.Cu") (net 6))
 (segment (start 112 95.54) (end 113.32 94.22) (width 0.5) (layer "F.Cu") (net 6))
 (segment (start 114.8 56.12) (end 113.06 56.12) (width 0.5) (layer "F.Cu") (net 6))
 (segment (start 93.22 94.2) (end 93.2 94.18) (width 0.5) (layer "F.Cu") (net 6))
 (segment (start 108.7 100.9) (end 110.7 100.9) (width 0.5) (layer "F.Cu") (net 6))
 (segment (start 113.32 94.22) (end 114.8 94.22) (width 0.5) (layer "F.Cu") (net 6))
 (segment (start 110.7 100.9) (end 112 99.6) (width 0.5) (layer "F.Cu") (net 6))
 (segment (start 118.42 95.62) (end 117.02 94.22) (width 0.5) (layer "F.Cu") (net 6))
 (segment (start 117.02 94.22) (end 114.8 94.22) (width 0.5) (layer "F.Cu") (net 6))
 (segment (start 114.8 63.74) (end 116.06 63.74) (width 0.5) (layer "F.Cu") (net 7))
 (segment (start 109.465 49.85) (end 110.715 48.6) (width 0.5) (layer "F.Cu") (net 7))
 (segment (start 117.3 62.5) (end 117.3 50.1) (width 0.5) (layer "F.Cu") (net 7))
 (segment (start 109.465 50.375) (end 109.465 49.85) (width 0.5) (layer "F.Cu") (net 7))
 (segment (start 117.3 50.1) (end 115.8 48.6) (width 0.5) (layer "F.Cu") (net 7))
 (segment (start 115.8 48.6) (end 110.715 48.6) (width 0.5) (layer "F.Cu") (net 7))
 (segment (start 116.06 63.74) (end 117.3 62.5) (width 0.5) (layer "F.Cu") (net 7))
 (segment (start 97.02 99.28) (end 93.22 99.28) (width 0.5) (layer "F.Cu") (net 22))
 (segment (start 93.22 99.28) (end 93.2 99.26) (width 0.5) (layer "F.Cu") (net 22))
 (segment (start 99.6 107.3) (end 99.6 102.8) (width 0.5) (layer "F.Cu") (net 26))
 (segment (start 115.88 102.8) (end 115.88 107.42) (width 0.5) (layer "F.Cu") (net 26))
 (segment (start 97.02 86.58) (end 98.2 86.58) (width 0.5) (layer "F.Cu") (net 26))
 (segment (start 114.4 108.9) (end 101.2 108.9) (width 0.5) (layer "F.Cu") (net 26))
 (segment (start 115.88 107.42) (end 114.4 108.9) (width 0.5) (layer "F.Cu") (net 26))
 (segment (start 99 101.3) (end 99 87.38) (width 0.5) (layer "F.Cu") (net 26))
 (segment (start 99 87.38) (end 98.2 86.58) (width 0.5) (layer "F.Cu") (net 26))
 (segment (start 101.2 108.9) (end 99.6 107.3) (width 0.5) (layer "F.Cu") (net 26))
 (segment (start 99.6 102.8) (end 99.6 101.9) (width 0.5) (layer "F.Cu") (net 26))
 (segment (start 99.6 101.9) (end 99 101.3) (width 0.5) (layer "F.Cu") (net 26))
 (segment (start 100.34 101) (end 100.3 101) (width 0.5) (layer "F.Cu") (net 27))
 (segment (start 100.3 101) (end 100.3 85.1) (width 0.5) (layer "F.Cu") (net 27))
 (segment (start 102.14 102.8) (end 100.34 101) (width 0.5) (layer "F.Cu") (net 27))
 (segment (start 113.34 106.26) (end 113.34 102.8) (width 0.5) (layer "F.Cu") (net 27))
 (segment (start 99.24 84.04) (end 97.02 84.04) (width 0.5) (layer "F.Cu") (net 27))
 (segment (start 112.3 107.3) (end 113.34 106.26) (width 0.5) (layer "F.Cu") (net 27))
 (segment (start 100.3 85.1) (end 99.24 84.04) (width 0.5) (layer "F.Cu") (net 27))
 (segment (start 102.14 102.8) (end 102.14 106.14) (width 0.5) (layer "F.Cu") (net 27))
 (segment (start 103.3 107.3) (end 112.3 107.3) (width 0.5) (layer "F.Cu") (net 27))
 (segment (start 102.14 106.14) (end 103.3 107.3) (width 0.5) (layer "F.Cu") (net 27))
 (segment (start 97.02 96.74) (end 93.22 96.74) (width 0.5) (layer "F.Cu") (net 23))
 (segment (start 93.22 96.74) (end 93.2 96.72) (width 0.5) (layer "F.Cu") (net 23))
 (segment (start 96.78 79.2) (end 96.1 79.2) (width 0.5) (layer "F.Cu") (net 28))
 (segment (start 95 80.3) (end 96.1 79.2) (width 0.5) (layer "F.Cu") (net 28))
 (segment (start 95 89.84) (end 95 80.3) (width 0.5) (layer "F.Cu") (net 28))
 (segment (start 93.2 91.64) (end 95 89.84) (width 0.5) (layer "F.Cu") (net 28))
 (segment (start 92.84 91.64) (end 93.2 91.64) (width 0.25) (layer "F.Cu") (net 28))
 (segment (start 97.02 78.96) (end 96.78 79.2) (width 0.5) (layer "F.Cu") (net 28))
 (segment (start 93.2 55.7) (end 94.85 54.05) (width 0.25) (layer "F.Cu") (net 34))
 (segment (start 93.2 55.7) (end 95.34 53.56) (width 0.5) (layer "F.Cu") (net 34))
 (segment (start 93.2 89.1) (end 93.2 55.7) (width 0.5) (layer "F.Cu") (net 34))
 (segment (start 97.02 53.56) (end 95.34 53.56) (width 0.5) (layer "F.Cu") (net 34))
 (segment (start 95.34 53.56) (end 94.85 54.05) (width 0.25) (layer "F.Cu") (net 34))
 (segment (start 94.85 54.05) (end 94.4 54.5) (width 0.25) (layer "F.Cu") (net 34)))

